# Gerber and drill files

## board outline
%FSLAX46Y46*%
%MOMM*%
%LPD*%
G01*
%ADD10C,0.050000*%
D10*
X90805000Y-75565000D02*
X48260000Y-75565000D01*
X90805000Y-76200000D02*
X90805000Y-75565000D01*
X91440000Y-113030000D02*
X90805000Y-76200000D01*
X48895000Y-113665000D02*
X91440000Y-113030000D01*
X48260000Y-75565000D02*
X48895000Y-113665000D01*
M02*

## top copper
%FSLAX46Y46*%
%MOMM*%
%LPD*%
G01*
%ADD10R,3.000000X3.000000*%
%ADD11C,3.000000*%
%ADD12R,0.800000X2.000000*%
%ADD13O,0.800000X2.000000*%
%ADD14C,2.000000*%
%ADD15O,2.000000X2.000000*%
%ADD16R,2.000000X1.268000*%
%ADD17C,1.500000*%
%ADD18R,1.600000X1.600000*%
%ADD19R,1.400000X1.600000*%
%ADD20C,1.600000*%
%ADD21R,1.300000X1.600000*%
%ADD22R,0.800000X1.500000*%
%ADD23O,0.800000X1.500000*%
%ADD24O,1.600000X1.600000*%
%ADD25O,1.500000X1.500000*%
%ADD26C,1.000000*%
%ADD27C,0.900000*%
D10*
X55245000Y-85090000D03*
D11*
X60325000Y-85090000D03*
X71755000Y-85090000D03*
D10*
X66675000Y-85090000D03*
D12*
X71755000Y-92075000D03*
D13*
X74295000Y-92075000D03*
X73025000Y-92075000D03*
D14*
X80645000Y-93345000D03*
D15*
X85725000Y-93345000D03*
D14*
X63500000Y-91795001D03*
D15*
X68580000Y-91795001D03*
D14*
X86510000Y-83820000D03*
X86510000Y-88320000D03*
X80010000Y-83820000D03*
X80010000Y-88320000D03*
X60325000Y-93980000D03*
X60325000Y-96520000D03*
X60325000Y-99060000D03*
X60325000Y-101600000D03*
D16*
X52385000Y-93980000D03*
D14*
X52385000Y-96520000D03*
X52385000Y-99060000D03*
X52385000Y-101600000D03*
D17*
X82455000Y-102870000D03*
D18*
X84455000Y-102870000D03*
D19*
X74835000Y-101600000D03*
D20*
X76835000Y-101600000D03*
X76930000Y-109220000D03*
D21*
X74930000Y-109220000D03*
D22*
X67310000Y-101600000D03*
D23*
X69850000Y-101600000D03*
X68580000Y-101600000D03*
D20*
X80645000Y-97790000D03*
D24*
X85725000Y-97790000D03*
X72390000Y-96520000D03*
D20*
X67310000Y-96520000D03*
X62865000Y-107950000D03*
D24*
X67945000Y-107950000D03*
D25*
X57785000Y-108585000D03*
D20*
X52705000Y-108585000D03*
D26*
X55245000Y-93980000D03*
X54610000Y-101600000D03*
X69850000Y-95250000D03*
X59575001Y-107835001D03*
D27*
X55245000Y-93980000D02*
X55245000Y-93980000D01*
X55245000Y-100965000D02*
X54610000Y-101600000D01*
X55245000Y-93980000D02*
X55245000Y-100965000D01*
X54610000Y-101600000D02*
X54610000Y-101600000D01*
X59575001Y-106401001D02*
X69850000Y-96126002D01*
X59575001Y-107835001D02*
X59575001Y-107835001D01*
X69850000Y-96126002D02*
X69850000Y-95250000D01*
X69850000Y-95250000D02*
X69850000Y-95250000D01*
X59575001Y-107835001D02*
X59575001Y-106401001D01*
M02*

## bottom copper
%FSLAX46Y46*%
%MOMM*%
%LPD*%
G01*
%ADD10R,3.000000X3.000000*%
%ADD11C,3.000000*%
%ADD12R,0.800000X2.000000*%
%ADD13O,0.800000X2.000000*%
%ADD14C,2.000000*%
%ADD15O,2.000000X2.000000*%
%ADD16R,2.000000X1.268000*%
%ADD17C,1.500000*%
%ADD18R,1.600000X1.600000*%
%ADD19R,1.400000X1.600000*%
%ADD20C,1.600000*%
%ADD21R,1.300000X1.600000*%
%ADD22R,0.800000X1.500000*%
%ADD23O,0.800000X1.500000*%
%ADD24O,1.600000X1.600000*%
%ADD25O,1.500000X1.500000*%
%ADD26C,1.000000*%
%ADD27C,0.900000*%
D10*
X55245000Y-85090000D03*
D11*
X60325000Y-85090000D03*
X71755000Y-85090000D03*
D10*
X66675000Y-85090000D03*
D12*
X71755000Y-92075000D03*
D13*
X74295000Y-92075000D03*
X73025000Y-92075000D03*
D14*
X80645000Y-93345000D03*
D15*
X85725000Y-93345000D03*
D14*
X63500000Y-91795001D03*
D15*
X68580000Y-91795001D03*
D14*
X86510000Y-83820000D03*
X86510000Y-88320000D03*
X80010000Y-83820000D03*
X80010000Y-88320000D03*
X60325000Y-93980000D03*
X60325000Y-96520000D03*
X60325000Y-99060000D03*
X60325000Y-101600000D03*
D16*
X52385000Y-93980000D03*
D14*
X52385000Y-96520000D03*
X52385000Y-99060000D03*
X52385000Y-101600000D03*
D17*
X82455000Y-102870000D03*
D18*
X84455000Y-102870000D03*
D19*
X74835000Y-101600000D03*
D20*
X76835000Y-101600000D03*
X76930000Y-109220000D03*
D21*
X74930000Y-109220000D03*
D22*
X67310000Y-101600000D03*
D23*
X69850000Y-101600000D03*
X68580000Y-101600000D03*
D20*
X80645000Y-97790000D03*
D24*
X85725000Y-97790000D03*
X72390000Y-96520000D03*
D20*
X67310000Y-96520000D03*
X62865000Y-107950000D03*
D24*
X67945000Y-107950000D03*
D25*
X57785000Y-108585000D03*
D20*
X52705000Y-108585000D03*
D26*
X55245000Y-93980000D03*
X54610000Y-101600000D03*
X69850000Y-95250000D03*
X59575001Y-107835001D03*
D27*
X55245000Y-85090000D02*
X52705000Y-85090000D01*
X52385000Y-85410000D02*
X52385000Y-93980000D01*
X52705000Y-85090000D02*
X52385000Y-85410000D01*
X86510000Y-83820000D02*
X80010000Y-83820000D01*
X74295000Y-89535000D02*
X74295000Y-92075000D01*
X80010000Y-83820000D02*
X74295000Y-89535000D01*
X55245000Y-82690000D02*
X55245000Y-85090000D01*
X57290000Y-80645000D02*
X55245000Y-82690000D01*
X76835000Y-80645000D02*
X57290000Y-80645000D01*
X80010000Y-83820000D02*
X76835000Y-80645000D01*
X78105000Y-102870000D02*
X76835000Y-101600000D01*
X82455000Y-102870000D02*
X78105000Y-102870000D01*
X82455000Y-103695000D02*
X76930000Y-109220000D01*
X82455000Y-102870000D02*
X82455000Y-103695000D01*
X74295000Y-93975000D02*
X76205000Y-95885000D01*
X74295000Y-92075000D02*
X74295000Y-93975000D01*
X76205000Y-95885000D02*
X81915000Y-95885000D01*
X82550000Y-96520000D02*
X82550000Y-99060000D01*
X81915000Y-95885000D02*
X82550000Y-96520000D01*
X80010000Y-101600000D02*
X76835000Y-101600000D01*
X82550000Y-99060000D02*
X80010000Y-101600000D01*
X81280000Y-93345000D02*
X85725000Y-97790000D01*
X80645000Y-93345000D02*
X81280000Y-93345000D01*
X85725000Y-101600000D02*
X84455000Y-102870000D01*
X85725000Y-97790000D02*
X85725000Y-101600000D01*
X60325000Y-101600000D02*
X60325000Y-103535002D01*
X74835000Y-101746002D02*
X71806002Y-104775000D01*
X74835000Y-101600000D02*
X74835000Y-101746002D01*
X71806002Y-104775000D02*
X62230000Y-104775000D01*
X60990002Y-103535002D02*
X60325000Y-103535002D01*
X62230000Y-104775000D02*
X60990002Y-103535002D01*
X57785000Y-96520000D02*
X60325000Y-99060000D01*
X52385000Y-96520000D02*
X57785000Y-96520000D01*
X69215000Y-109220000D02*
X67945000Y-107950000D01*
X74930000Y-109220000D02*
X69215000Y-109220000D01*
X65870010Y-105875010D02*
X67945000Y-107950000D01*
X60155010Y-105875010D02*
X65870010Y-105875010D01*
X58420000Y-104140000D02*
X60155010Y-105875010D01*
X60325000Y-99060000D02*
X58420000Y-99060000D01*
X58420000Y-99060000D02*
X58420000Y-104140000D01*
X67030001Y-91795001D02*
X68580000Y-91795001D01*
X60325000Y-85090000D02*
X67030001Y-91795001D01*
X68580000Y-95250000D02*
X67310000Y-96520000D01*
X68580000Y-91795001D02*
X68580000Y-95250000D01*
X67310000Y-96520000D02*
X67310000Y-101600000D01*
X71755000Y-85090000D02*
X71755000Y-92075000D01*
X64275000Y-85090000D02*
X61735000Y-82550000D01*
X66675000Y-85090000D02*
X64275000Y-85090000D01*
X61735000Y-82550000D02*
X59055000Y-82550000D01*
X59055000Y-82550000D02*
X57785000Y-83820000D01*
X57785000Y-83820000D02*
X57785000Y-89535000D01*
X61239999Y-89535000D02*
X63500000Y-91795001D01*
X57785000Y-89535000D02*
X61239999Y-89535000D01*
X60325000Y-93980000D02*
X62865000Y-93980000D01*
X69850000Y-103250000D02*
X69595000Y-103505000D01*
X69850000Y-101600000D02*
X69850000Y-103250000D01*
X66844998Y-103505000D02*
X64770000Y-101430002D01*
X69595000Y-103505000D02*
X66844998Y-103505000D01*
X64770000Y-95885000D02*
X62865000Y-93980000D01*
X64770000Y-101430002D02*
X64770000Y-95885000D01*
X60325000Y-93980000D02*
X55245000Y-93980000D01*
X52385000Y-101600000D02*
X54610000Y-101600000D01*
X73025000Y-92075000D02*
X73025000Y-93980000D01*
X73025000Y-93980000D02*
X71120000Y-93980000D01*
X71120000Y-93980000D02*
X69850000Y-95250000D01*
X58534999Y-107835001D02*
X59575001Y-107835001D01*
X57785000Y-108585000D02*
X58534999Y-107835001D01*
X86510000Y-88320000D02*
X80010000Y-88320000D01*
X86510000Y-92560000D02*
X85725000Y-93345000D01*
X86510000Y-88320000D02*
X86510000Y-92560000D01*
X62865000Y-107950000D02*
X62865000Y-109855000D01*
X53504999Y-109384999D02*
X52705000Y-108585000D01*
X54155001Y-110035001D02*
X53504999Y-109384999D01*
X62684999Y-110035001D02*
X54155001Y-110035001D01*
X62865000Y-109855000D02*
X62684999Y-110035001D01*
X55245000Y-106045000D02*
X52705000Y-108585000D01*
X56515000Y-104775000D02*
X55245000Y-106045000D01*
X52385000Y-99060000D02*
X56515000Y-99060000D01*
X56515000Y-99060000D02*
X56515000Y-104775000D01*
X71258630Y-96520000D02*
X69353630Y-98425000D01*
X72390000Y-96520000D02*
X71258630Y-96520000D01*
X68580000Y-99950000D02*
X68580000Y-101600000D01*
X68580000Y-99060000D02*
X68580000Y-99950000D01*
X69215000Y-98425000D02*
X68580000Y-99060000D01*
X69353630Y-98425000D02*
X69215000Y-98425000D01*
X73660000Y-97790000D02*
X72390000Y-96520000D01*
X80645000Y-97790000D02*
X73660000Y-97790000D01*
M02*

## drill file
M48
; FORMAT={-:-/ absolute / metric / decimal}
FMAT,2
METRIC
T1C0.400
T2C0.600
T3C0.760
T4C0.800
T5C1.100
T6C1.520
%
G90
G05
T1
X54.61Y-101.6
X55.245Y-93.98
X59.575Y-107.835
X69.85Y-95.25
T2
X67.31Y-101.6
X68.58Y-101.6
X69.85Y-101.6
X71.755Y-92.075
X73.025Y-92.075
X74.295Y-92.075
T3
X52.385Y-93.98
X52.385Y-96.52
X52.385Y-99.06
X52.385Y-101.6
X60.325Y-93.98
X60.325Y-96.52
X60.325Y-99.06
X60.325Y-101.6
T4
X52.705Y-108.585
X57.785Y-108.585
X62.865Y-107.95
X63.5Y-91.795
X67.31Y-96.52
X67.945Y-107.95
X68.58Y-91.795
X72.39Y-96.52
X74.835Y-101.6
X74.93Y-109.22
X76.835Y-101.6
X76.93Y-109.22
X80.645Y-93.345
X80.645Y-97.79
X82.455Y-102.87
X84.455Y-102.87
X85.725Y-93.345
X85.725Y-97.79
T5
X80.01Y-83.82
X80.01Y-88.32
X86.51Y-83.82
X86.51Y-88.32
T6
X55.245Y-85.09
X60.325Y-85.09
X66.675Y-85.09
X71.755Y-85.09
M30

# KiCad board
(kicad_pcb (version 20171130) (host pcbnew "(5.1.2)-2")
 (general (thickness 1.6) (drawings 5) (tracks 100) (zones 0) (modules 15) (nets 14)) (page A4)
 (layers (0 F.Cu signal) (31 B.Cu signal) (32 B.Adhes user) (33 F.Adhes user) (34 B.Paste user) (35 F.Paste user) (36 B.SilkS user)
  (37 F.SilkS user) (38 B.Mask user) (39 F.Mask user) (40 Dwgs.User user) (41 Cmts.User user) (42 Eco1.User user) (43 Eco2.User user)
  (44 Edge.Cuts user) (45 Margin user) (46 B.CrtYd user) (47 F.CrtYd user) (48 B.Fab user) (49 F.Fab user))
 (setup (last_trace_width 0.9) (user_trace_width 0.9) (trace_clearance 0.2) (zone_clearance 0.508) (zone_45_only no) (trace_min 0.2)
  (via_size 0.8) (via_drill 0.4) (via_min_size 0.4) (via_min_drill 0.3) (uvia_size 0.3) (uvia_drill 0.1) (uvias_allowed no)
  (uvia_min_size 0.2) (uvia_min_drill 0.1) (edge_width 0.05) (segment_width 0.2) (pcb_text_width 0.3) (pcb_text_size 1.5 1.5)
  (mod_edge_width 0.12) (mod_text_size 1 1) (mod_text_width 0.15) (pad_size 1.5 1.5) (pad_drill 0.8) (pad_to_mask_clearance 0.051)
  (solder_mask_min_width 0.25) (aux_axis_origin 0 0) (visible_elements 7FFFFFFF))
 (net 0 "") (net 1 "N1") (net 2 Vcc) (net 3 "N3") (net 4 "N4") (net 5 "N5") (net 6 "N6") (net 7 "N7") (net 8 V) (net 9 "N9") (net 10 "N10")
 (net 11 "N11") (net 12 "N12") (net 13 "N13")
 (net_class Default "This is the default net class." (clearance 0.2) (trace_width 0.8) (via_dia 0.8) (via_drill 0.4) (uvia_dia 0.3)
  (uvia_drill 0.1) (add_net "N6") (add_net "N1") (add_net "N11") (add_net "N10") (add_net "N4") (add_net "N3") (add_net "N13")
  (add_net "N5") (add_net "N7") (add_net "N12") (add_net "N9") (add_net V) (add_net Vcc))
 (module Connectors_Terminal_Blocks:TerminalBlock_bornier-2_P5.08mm (layer F.Cu) (at 55.245 85.09)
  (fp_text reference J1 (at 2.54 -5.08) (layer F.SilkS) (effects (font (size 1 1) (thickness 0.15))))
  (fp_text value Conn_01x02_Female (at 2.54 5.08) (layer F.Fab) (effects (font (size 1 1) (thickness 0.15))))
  (pad 1 thru_hole rect (at 0 0) (size 3 3) (drill 1.52) (layers *.Cu *.Mask) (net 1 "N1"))
  (pad 2 thru_hole circle (at 5.08 0) (size 3 3) (drill 1.52) (layers *.Cu *.Mask) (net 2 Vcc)))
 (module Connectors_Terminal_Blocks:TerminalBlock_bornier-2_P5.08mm (layer F.Cu) (at 66.675 85.09)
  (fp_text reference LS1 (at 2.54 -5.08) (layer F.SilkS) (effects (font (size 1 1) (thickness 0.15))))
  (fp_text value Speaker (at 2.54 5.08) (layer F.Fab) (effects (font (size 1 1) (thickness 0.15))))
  (pad 2 thru_hole circle (at 5.08 0) (size 3 3) (drill 1.52) (layers *.Cu *.Mask) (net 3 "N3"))
  (pad 1 thru_hole rect (at 0 0) (size 3 3) (drill 1.52) (layers *.Cu *.Mask) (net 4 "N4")))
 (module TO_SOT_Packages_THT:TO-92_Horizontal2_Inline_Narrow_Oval (layer F.Cu) (at 71.755 92.075)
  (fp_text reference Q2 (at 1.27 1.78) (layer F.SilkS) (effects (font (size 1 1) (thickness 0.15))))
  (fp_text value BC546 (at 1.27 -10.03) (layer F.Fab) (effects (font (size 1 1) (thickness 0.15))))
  (pad 1 thru_hole rect (at 0 0 180) (size 0.8 2) (drill 0.6) (layers *.Cu *.Mask) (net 3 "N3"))
  (pad 3 thru_hole oval (at 2.54 0 180) (size 0.8 2) (drill 0.6) (layers *.Cu *.Mask) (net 1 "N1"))
  (pad 2 thru_hole oval (at 1.27 0 180) (size 0.8 2) (drill 0.6) (layers *.Cu *.Mask) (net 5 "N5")))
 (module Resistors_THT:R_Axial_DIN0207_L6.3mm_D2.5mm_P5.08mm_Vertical (layer F.Cu) (at 80.645 93.345)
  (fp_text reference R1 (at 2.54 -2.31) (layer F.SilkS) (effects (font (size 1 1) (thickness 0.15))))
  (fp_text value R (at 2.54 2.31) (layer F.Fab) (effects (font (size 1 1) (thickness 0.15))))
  (pad 1 thru_hole circle (at 0 0) (size 2 2) (drill 0.8) (layers *.Cu *.Mask) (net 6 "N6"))
  (pad 2 thru_hole oval (at 5.08 0) (size 2 2) (drill 0.8) (layers *.Cu *.Mask) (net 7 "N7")))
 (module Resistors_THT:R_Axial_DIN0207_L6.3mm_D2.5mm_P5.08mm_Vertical (layer F.Cu) (at 63.5 91.795001)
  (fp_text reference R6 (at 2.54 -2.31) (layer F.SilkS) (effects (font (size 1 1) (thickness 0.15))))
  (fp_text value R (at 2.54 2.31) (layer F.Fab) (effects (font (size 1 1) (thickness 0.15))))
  (pad 1 thru_hole circle (at 0 0) (size 2 2) (drill 0.8) (layers *.Cu *.Mask) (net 4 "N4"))
  (pad 2 thru_hole oval (at 5.08 0) (size 2 2) (drill 0.8) (layers *.Cu *.Mask) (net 2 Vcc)))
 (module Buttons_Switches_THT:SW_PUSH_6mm (layer F.Cu) (at 80.01 83.82)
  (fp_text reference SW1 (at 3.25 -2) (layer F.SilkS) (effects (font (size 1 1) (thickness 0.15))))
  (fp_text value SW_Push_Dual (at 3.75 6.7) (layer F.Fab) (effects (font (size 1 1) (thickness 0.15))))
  (pad 1 thru_hole circle (at 6.5 0 90) (size 2 2) (drill 1.1) (layers *.Cu *.Mask) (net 1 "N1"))
  (pad 2 thru_hole circle (at 6.5 4.5 90) (size 2 2) (drill 1.1) (layers *.Cu *.Mask) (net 7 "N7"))
  (pad 1 thru_hole circle (at 0 0 90) (size 2 2) (drill 1.1) (layers *.Cu *.Mask) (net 1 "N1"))
  (pad 2 thru_hole circle (at 0 4.5 90) (size 2 2) (drill 1.1) (layers *.Cu *.Mask) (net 7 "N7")))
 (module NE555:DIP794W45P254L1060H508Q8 (layer F.Cu) (at 56.355 97.79)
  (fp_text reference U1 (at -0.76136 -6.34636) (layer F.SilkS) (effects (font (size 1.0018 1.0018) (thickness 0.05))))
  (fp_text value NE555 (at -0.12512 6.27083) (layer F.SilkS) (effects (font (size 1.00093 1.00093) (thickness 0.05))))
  (pad 8 thru_hole circle (at 3.97 -3.81 270) (size 2 2) (drill 0.76) (layers *.Cu *.Mask) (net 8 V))
  (pad 7 thru_hole circle (at 3.97 -1.27 270) (size 2 2) (drill 0.76) (layers *.Cu *.Mask) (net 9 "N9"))
  (pad 6 thru_hole circle (at 3.97 1.27 270) (size 2 2) (drill 0.76) (layers *.Cu *.Mask) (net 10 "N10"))
  (pad 5 thru_hole circle (at 3.97 3.81 270) (size 2 2) (drill 0.76) (layers *.Cu *.Mask) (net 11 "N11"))
  (pad 1 thru_hole rect (at -3.97 -3.81 270) (size 1.268 2) (drill 0.76) (layers *.Cu *.Mask) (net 1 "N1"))
  (pad 2 thru_hole circle (at -3.97 -1.27 270) (size 2 2) (drill 0.76) (layers *.Cu *.Mask) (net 10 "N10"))
  (pad 3 thru_hole circle (at -3.97 1.27 270) (size 2 2) (drill 0.76) (layers *.Cu *.Mask) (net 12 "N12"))
  (pad 4 thru_hole circle (at -3.97 3.81 270) (size 2 2) (drill 0.76) (layers *.Cu *.Mask) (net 8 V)))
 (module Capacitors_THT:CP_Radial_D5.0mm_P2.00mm (layer F.Cu) (at 84.455 102.87 180)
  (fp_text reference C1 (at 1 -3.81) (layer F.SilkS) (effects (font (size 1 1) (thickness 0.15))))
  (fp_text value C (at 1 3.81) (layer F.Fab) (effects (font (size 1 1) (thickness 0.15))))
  (pad 2 thru_hole circle (at 2 0 180) (size 1.5 1.5) (drill 0.8) (layers *.Cu *.Mask) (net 1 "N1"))
  (pad 1 thru_hole rect (at 0 0 180) (size 1.6 1.6) (drill 0.8) (layers *.Cu *.Mask) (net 6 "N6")))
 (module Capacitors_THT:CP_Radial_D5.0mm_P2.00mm (layer F.Cu) (at 74.835 101.6)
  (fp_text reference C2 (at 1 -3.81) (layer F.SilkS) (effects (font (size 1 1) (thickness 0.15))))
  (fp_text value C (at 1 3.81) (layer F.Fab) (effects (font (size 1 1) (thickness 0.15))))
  (pad 1 thru_hole rect (at 0 0) (size 1.4 1.6) (drill 0.8) (layers *.Cu *.Mask) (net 11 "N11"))
  (pad 2 thru_hole circle (at 2 0) (size 1.6 1.6) (drill 0.8) (layers *.Cu *.Mask) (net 1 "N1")))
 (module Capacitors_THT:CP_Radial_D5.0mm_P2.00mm (layer F.Cu) (at 74.93 109.22)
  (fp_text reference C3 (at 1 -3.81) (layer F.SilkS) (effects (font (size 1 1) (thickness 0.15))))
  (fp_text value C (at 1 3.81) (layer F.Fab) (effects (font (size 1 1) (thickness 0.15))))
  (pad 2 thru_hole circle (at 2 0) (size 1.6 1.6) (drill 0.8) (layers *.Cu *.Mask) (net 1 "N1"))
  (pad 1 thru_hole rect (at 0 0) (size 1.3 1.6) (drill 0.8) (layers *.Cu *.Mask) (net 10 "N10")))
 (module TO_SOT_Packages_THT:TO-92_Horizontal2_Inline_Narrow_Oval (layer F.Cu) (at 67.31 101.6)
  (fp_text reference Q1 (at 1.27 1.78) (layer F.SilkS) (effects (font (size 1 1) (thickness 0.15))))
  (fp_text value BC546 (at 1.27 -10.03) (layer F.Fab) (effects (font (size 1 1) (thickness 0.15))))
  (pad 1 thru_hole rect (at 0 0 180) (size 0.8 1.5) (drill 0.6) (layers *.Cu *.Mask) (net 2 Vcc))
  (pad 3 thru_hole oval (at 2.54 0 180) (size 0.8 1.5) (drill 0.6) (layers *.Cu *.Mask) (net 8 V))
  (pad 2 thru_hole oval (at 1.27 0 180) (size 0.8 1.5) (drill 0.6) (layers *.Cu *.Mask) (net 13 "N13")))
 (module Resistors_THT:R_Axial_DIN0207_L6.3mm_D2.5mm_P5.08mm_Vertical (layer F.Cu) (at 80.645 97.79)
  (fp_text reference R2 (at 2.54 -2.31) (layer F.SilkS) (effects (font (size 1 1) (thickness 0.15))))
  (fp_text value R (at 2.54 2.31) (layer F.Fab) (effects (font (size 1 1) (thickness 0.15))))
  (pad 1 thru_hole circle (at 0 0) (size 1.6 1.6) (drill 0.8) (layers *.Cu *.Mask) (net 13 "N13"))
  (pad 2 thru_hole oval (at 5.08 0) (size 1.6 1.6) (drill 0.8) (layers *.Cu *.Mask) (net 6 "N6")))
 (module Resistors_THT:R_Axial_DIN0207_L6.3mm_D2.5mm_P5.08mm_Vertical (layer F.Cu) (at 67.31 96.52)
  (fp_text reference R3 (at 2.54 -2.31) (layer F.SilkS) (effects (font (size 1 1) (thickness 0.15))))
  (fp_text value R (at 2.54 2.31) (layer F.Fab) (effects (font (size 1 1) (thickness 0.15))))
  (pad 2 thru_hole oval (at 5.08 0) (size 1.6 1.6) (drill 0.8) (layers *.Cu *.Mask) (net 13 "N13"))
  (pad 1 thru_hole circle (at 0 0) (size 1.6 1.6) (drill 0.8) (layers *.Cu *.Mask) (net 2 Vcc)))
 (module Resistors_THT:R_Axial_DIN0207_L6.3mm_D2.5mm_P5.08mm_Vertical (layer F.Cu) (at 62.865 107.95)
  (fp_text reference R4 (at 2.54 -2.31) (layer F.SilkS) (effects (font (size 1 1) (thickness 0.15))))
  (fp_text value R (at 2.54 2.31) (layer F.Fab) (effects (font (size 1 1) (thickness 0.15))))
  (pad 1 thru_hole circle (at 0 0) (size 1.6 1.6) (drill 0.8) (layers *.Cu *.Mask) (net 12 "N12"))
  (pad 2 thru_hole oval (at 5.08 0) (size 1.6 1.6) (drill 0.8) (layers *.Cu *.Mask) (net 10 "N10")))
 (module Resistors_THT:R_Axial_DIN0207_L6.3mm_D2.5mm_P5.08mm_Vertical (layer F.Cu) (at 52.705 108.585)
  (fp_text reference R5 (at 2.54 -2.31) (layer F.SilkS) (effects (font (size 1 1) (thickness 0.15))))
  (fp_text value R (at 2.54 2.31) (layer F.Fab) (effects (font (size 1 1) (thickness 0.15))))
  (pad 2 thru_hole oval (at 5.08 0) (size 1.5 1.5) (drill 0.8) (layers *.Cu *.Mask) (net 5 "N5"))
  (pad 1 thru_hole circle (at 0 0) (size 1.6 1.6) (drill 0.8) (layers *.Cu *.Mask) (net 12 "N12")))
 (gr_line (start 90.805 75.565) (end 48.26 75.565) (layer Edge.Cuts) (width 0.05))
 (gr_line (start 90.805 76.2) (end 90.805 75.565) (layer Edge.Cuts) (width 0.05))
 (gr_line (start 91.44 113.03) (end 90.805 76.2) (layer Edge.Cuts) (width 0.05))
 (gr_line (start 48.895 113.665) (end 91.44 113.03) (layer Edge.Cuts) (width 0.05))
 (gr_line (start 48.26 75.565) (end 48.895 113.665) (layer Edge.Cuts) (width 0.05))
 (segment (start 55.245 85.09) (end 52.705 85.09) (width 0.9) (layer B.Cu) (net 1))
 (segment (start 52.385 85.41) (end 52.385 93.98) (width 0.9) (layer B.Cu) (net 1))
 (segment (start 52.705 85.09) (end 52.385 85.41) (width 0.9) (layer B.Cu) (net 1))
 (segment (start 86.51 83.82) (end 80.01 83.82) (width 0.9) (layer B.Cu) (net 1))
 (segment (start 74.295 89.535) (end 74.295 92.075) (width 0.9) (layer B.Cu) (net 1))
 (segment (start 80.01 83.82) (end 74.295 89.535) (width 0.9) (layer B.Cu) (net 1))
 (segment (start 55.245 82.69) (end 55.245 85.09) (width 0.9) (layer B.Cu) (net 1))
 (segment (start 57.29 80.645) (end 55.245 82.69) (width 0.9) (layer B.Cu) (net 1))
 (segment (start 76.835 80.645) (end 57.29 80.645) (width 0.9) (layer B.Cu) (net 1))
 (segment (start 80.01 83.82) (end 76.835 80.645) (width 0.9) (layer B.Cu) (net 1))
 (segment (start 78.105 102.87) (end 76.835 101.6) (width 0.9) (layer B.Cu) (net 1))
 (segment (start 82.455 102.87) (end 78.105 102.87) (width 0.9) (layer B.Cu) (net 1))
 (segment (start 82.455 103.695) (end 76.93 109.22) (width 0.9) (layer B.Cu) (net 1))
 (segment (start 82.455 102.87) (end 82.455 103.695) (width 0.9) (layer B.Cu) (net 1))
 (segment (start 74.295 93.975) (end 76.205 95.885) (width 0.9) (layer B.Cu) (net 1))
 (segment (start 74.295 92.075) (end 74.295 93.975) (width 0.9) (layer B.Cu) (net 1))
 (segment (start 76.205 95.885) (end 81.915 95.885) (width 0.9) (layer B.Cu) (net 1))
 (segment (start 82.55 96.52) (end 82.55 99.06) (width 0.9) (layer B.Cu) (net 1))
 (segment (start 81.915 95.885) (end 82.55 96.52) (width 0.9) (layer B.Cu) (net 1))
 (segment (start 80.01 101.6) (end 76.835 101.6) (width 0.9) (layer B.Cu) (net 1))
 (segment (start 82.55 99.06) (end 80.01 101.6) (width 0.9) (layer B.Cu) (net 1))
 (segment (start 81.28 93.345) (end 85.725 97.79) (width 0.9) (layer B.Cu) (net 6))
 (segment (start 80.645 93.345) (end 81.28 93.345) (width 0.9) (layer B.Cu) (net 6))
 (segment (start 85.725 101.6) (end 84.455 102.87) (width 0.9) (layer B.Cu) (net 6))
 (segment (start 85.725 97.79) (end 85.725 101.6) (width 0.9) (layer B.Cu) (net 6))
 (segment (start 60.325 101.6) (end 60.325 103.535002) (width 0.9) (layer B.Cu) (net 11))
 (segment (start 74.835 101.746002) (end 71.806002 104.775) (width 0.9) (layer B.Cu) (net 11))
 (segment (start 74.835 101.6) (end 74.835 101.746002) (width 0.9) (layer B.Cu) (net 11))
 (segment (start 71.806002 104.775) (end 62.23 104.775) (width 0.9) (layer B.Cu) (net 11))
 (segment (start 60.990002 103.535002) (end 60.325 103.535002) (width 0.9) (layer B.Cu) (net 11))
 (segment (start 62.23 104.775) (end 60.990002 103.535002) (width 0.9) (layer B.Cu) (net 11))
 (segment (start 57.785 96.52) (end 60.325 99.06) (width 0.9) (layer B.Cu) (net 10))
 (segment (start 52.385 96.52) (end 57.785 96.52) (width 0.9) (layer B.Cu) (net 10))
 (segment (start 69.215 109.22) (end 67.945 107.95) (width 0.9) (layer B.Cu) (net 10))
 (segment (start 74.93 109.22) (end 69.215 109.22) (width 0.9) (layer B.Cu) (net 10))
 (segment (start 65.87001 105.87501) (end 67.945 107.95) (width 0.9) (layer B.Cu) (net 10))
 (segment (start 60.15501 105.87501) (end 65.87001 105.87501) (width 0.9) (layer B.Cu) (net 10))
 (segment (start 58.42 104.14) (end 60.15501 105.87501) (width 0.9) (layer B.Cu) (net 10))
 (segment (start 60.325 99.06) (end 58.42 99.06) (width 0.9) (layer B.Cu) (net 10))
 (segment (start 58.42 99.06) (end 58.42 104.14) (width 0.9) (layer B.Cu) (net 10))
 (segment (start 67.030001 91.795001) (end 68.58 91.795001) (width 0.9) (layer B.Cu) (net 2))
 (segment (start 60.325 85.09) (end 67.030001 91.795001) (width 0.9) (layer B.Cu) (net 2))
 (segment (start 68.58 95.25) (end 67.31 96.52) (width 0.9) (layer B.Cu) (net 2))
 (segment (start 68.58 91.795001) (end 68.58 95.25) (width 0.9) (layer B.Cu) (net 2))
 (segment (start 67.31 96.52) (end 67.31 101.6) (width 0.9) (layer B.Cu) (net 2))
 (segment (start 71.755 85.09) (end 71.755 92.075) (width 0.9) (layer B.Cu) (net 3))
 (segment (start 64.275 85.09) (end 61.735 82.55) (width 0.9) (layer B.Cu) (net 4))
 (segment (start 66.675 85.09) (end 64.275 85.09) (width 0.9) (layer B.Cu) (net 4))
 (segment (start 61.735 82.55) (end 59.055 82.55) (width 0.9) (layer B.Cu) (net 4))
 (segment (start 59.055 82.55) (end 57.785 83.82) (width 0.9) (layer B.Cu) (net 4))
 (segment (start 57.785 83.82) (end 57.785 89.535) (width 0.9) (layer B.Cu) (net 4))
 (segment (start 61.239999 89.535) (end 63.5 91.795001) (width 0.9) (layer B.Cu) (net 4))
 (segment (start 57.785 89.535) (end 61.239999 89.535) (width 0.9) (layer B.Cu) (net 4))
 (segment (start 60.325 93.98) (end 62.865 93.98) (width 0.9) (layer B.Cu) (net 8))
 (segment (start 69.85 103.25) (end 69.595 103.505) (width 0.9) (layer B.Cu) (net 8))
 (segment (start 69.85 101.6) (end 69.85 103.25) (width 0.9) (layer B.Cu) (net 8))
 (segment (start 66.844998 103.505) (end 64.77 101.430002) (width 0.9) (layer B.Cu) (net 8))
 (segment (start 69.595 103.505) (end 66.844998 103.505) (width 0.9) (layer B.Cu) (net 8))
 (segment (start 64.77 95.885) (end 62.865 93.98) (width 0.9) (layer B.Cu) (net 8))
 (segment (start 64.77 101.430002) (end 64.77 95.885) (width 0.9) (layer B.Cu) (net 8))
 (segment (start 60.325 93.98) (end 55.245 93.98) (width 0.9) (layer B.Cu) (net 8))
 (segment (start 52.385 101.6) (end 54.61 101.6) (width 0.9) (layer B.Cu) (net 8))
 (segment (start 55.245 93.98) (end 55.245 93.98) (width 0.9) (layer F.Cu) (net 8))
 (segment (start 55.245 100.965) (end 54.61 101.6) (width 0.9) (layer F.Cu) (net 8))
 (segment (start 55.245 93.98) (end 55.245 100.965) (width 0.9) (layer F.Cu) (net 8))
 (via (at 55.245 93.98) (size 1) (drill 0.4) (layers F.Cu B.Cu) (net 8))
 (segment (start 54.61 101.6) (end 54.61 101.6) (width 0.9) (layer F.Cu) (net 8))
 (via (at 54.61 101.6) (size 1) (drill 0.4) (layers F.Cu B.Cu) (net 8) (status 1000000))
 (segment (start 73.025 92.075) (end 73.025 93.98) (width 0.9) (layer B.Cu) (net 5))
 (segment (start 73.025 93.98) (end 71.12 93.98) (width 0.9) (layer B.Cu) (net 5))
 (segment (start 71.12 93.98) (end 69.85 95.25) (width 0.9) (layer B.Cu) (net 5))
 (segment (start 58.534999 107.835001) (end 59.575001 107.835001) (width 0.9) (layer B.Cu) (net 5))
 (segment (start 57.785 108.585) (end 58.534999 107.835001) (width 0.9) (layer B.Cu) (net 5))
 (segment (start 59.575001 106.401001) (end 69.85 96.126002) (width 0.9) (layer F.Cu) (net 5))
 (segment (start 59.575001 107.835001) (end 59.575001 107.835001) (width 0.9) (layer F.Cu) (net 5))
 (segment (start 69.85 96.126002) (end 69.85 95.25) (width 0.9) (layer F.Cu) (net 5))
 (segment (start 69.85 95.25) (end 69.85 95.25) (width 0.9) (layer F.Cu) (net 5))
 (via (at 69.85 95.25) (size 1) (drill 0.4) (layers F.Cu B.Cu) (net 5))
 (segment (start 59.575001 107.835001) (end 59.575001 106.401001) (width 0.9) (layer F.Cu) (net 5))
 (via (at 59.575001 107.835001) (size 1) (drill 0.4) (layers F.Cu B.Cu) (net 5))
 (segment (start 86.51 88.32) (end 80.01 88.32) (width 0.9) (layer B.Cu) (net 7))
 (segment (start 86.51 92.56) (end 85.725 93.345) (width 0.9) (layer B.Cu) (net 7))
 (segment (start 86.51 88.32) (end 86.51 92.56) (width 0.9) (layer B.Cu) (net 7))
 (segment (start 62.865 107.95) (end 62.865 109.855) (width 0.9) (layer B.Cu) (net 12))
 (segment (start 53.504999 109.384999) (end 52.705 108.585) (width 0.9) (layer B.Cu) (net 12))
 (segment (start 54.155001 110.035001) (end 53.504999 109.384999) (width 0.9) (layer B.Cu) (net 12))
 (segment (start 62.684999 110.035001) (end 54.155001 110.035001) (width 0.9) (layer B.Cu) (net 12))
 (segment (start 62.865 109.855) (end 62.684999 110.035001) (width 0.9) (layer B.Cu) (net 12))
 (segment (start 55.245 106.045) (end 52.705 108.585) (width 0.9) (layer B.Cu) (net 12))
 (segment (start 56.515 104.775) (end 55.245 106.045) (width 0.9) (layer B.Cu) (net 12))
 (segment (start 52.385 99.06) (end 56.515 99.06) (width 0.9) (layer B.Cu) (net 12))
 (segment (start 56.515 99.06) (end 56.515 104.775) (width 0.9) (layer B.Cu) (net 12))
 (segment (start 71.25863 96.52) (end 69.35363 98.425) (width 0.9) (layer B.Cu) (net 13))
 (segment (start 72.39 96.52) (end 71.25863 96.52) (width 0.9) (layer B.Cu) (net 13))
 (segment (start 68.58 99.95) (end 68.58 101.6) (width 0.9) (layer B.Cu) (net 13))
 (segment (start 68.58 99.06) (end 68.58 99.95) (width 0.9) (layer B.Cu) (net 13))
 (segment (start 69.215 98.425) (end 68.58 99.06) (width 0.9) (layer B.Cu) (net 13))
 (segment (start 69.35363 98.425) (end 69.215 98.425) (width 0.9) (layer B.Cu) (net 13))
 (segment (start 73.66 97.79) (end 72.39 96.52) (width 0.9) (layer B.Cu) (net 13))
 (segment (start 80.645 97.79) (end 73.66 97.79) (width 0.9) (layer B.Cu) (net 13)))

